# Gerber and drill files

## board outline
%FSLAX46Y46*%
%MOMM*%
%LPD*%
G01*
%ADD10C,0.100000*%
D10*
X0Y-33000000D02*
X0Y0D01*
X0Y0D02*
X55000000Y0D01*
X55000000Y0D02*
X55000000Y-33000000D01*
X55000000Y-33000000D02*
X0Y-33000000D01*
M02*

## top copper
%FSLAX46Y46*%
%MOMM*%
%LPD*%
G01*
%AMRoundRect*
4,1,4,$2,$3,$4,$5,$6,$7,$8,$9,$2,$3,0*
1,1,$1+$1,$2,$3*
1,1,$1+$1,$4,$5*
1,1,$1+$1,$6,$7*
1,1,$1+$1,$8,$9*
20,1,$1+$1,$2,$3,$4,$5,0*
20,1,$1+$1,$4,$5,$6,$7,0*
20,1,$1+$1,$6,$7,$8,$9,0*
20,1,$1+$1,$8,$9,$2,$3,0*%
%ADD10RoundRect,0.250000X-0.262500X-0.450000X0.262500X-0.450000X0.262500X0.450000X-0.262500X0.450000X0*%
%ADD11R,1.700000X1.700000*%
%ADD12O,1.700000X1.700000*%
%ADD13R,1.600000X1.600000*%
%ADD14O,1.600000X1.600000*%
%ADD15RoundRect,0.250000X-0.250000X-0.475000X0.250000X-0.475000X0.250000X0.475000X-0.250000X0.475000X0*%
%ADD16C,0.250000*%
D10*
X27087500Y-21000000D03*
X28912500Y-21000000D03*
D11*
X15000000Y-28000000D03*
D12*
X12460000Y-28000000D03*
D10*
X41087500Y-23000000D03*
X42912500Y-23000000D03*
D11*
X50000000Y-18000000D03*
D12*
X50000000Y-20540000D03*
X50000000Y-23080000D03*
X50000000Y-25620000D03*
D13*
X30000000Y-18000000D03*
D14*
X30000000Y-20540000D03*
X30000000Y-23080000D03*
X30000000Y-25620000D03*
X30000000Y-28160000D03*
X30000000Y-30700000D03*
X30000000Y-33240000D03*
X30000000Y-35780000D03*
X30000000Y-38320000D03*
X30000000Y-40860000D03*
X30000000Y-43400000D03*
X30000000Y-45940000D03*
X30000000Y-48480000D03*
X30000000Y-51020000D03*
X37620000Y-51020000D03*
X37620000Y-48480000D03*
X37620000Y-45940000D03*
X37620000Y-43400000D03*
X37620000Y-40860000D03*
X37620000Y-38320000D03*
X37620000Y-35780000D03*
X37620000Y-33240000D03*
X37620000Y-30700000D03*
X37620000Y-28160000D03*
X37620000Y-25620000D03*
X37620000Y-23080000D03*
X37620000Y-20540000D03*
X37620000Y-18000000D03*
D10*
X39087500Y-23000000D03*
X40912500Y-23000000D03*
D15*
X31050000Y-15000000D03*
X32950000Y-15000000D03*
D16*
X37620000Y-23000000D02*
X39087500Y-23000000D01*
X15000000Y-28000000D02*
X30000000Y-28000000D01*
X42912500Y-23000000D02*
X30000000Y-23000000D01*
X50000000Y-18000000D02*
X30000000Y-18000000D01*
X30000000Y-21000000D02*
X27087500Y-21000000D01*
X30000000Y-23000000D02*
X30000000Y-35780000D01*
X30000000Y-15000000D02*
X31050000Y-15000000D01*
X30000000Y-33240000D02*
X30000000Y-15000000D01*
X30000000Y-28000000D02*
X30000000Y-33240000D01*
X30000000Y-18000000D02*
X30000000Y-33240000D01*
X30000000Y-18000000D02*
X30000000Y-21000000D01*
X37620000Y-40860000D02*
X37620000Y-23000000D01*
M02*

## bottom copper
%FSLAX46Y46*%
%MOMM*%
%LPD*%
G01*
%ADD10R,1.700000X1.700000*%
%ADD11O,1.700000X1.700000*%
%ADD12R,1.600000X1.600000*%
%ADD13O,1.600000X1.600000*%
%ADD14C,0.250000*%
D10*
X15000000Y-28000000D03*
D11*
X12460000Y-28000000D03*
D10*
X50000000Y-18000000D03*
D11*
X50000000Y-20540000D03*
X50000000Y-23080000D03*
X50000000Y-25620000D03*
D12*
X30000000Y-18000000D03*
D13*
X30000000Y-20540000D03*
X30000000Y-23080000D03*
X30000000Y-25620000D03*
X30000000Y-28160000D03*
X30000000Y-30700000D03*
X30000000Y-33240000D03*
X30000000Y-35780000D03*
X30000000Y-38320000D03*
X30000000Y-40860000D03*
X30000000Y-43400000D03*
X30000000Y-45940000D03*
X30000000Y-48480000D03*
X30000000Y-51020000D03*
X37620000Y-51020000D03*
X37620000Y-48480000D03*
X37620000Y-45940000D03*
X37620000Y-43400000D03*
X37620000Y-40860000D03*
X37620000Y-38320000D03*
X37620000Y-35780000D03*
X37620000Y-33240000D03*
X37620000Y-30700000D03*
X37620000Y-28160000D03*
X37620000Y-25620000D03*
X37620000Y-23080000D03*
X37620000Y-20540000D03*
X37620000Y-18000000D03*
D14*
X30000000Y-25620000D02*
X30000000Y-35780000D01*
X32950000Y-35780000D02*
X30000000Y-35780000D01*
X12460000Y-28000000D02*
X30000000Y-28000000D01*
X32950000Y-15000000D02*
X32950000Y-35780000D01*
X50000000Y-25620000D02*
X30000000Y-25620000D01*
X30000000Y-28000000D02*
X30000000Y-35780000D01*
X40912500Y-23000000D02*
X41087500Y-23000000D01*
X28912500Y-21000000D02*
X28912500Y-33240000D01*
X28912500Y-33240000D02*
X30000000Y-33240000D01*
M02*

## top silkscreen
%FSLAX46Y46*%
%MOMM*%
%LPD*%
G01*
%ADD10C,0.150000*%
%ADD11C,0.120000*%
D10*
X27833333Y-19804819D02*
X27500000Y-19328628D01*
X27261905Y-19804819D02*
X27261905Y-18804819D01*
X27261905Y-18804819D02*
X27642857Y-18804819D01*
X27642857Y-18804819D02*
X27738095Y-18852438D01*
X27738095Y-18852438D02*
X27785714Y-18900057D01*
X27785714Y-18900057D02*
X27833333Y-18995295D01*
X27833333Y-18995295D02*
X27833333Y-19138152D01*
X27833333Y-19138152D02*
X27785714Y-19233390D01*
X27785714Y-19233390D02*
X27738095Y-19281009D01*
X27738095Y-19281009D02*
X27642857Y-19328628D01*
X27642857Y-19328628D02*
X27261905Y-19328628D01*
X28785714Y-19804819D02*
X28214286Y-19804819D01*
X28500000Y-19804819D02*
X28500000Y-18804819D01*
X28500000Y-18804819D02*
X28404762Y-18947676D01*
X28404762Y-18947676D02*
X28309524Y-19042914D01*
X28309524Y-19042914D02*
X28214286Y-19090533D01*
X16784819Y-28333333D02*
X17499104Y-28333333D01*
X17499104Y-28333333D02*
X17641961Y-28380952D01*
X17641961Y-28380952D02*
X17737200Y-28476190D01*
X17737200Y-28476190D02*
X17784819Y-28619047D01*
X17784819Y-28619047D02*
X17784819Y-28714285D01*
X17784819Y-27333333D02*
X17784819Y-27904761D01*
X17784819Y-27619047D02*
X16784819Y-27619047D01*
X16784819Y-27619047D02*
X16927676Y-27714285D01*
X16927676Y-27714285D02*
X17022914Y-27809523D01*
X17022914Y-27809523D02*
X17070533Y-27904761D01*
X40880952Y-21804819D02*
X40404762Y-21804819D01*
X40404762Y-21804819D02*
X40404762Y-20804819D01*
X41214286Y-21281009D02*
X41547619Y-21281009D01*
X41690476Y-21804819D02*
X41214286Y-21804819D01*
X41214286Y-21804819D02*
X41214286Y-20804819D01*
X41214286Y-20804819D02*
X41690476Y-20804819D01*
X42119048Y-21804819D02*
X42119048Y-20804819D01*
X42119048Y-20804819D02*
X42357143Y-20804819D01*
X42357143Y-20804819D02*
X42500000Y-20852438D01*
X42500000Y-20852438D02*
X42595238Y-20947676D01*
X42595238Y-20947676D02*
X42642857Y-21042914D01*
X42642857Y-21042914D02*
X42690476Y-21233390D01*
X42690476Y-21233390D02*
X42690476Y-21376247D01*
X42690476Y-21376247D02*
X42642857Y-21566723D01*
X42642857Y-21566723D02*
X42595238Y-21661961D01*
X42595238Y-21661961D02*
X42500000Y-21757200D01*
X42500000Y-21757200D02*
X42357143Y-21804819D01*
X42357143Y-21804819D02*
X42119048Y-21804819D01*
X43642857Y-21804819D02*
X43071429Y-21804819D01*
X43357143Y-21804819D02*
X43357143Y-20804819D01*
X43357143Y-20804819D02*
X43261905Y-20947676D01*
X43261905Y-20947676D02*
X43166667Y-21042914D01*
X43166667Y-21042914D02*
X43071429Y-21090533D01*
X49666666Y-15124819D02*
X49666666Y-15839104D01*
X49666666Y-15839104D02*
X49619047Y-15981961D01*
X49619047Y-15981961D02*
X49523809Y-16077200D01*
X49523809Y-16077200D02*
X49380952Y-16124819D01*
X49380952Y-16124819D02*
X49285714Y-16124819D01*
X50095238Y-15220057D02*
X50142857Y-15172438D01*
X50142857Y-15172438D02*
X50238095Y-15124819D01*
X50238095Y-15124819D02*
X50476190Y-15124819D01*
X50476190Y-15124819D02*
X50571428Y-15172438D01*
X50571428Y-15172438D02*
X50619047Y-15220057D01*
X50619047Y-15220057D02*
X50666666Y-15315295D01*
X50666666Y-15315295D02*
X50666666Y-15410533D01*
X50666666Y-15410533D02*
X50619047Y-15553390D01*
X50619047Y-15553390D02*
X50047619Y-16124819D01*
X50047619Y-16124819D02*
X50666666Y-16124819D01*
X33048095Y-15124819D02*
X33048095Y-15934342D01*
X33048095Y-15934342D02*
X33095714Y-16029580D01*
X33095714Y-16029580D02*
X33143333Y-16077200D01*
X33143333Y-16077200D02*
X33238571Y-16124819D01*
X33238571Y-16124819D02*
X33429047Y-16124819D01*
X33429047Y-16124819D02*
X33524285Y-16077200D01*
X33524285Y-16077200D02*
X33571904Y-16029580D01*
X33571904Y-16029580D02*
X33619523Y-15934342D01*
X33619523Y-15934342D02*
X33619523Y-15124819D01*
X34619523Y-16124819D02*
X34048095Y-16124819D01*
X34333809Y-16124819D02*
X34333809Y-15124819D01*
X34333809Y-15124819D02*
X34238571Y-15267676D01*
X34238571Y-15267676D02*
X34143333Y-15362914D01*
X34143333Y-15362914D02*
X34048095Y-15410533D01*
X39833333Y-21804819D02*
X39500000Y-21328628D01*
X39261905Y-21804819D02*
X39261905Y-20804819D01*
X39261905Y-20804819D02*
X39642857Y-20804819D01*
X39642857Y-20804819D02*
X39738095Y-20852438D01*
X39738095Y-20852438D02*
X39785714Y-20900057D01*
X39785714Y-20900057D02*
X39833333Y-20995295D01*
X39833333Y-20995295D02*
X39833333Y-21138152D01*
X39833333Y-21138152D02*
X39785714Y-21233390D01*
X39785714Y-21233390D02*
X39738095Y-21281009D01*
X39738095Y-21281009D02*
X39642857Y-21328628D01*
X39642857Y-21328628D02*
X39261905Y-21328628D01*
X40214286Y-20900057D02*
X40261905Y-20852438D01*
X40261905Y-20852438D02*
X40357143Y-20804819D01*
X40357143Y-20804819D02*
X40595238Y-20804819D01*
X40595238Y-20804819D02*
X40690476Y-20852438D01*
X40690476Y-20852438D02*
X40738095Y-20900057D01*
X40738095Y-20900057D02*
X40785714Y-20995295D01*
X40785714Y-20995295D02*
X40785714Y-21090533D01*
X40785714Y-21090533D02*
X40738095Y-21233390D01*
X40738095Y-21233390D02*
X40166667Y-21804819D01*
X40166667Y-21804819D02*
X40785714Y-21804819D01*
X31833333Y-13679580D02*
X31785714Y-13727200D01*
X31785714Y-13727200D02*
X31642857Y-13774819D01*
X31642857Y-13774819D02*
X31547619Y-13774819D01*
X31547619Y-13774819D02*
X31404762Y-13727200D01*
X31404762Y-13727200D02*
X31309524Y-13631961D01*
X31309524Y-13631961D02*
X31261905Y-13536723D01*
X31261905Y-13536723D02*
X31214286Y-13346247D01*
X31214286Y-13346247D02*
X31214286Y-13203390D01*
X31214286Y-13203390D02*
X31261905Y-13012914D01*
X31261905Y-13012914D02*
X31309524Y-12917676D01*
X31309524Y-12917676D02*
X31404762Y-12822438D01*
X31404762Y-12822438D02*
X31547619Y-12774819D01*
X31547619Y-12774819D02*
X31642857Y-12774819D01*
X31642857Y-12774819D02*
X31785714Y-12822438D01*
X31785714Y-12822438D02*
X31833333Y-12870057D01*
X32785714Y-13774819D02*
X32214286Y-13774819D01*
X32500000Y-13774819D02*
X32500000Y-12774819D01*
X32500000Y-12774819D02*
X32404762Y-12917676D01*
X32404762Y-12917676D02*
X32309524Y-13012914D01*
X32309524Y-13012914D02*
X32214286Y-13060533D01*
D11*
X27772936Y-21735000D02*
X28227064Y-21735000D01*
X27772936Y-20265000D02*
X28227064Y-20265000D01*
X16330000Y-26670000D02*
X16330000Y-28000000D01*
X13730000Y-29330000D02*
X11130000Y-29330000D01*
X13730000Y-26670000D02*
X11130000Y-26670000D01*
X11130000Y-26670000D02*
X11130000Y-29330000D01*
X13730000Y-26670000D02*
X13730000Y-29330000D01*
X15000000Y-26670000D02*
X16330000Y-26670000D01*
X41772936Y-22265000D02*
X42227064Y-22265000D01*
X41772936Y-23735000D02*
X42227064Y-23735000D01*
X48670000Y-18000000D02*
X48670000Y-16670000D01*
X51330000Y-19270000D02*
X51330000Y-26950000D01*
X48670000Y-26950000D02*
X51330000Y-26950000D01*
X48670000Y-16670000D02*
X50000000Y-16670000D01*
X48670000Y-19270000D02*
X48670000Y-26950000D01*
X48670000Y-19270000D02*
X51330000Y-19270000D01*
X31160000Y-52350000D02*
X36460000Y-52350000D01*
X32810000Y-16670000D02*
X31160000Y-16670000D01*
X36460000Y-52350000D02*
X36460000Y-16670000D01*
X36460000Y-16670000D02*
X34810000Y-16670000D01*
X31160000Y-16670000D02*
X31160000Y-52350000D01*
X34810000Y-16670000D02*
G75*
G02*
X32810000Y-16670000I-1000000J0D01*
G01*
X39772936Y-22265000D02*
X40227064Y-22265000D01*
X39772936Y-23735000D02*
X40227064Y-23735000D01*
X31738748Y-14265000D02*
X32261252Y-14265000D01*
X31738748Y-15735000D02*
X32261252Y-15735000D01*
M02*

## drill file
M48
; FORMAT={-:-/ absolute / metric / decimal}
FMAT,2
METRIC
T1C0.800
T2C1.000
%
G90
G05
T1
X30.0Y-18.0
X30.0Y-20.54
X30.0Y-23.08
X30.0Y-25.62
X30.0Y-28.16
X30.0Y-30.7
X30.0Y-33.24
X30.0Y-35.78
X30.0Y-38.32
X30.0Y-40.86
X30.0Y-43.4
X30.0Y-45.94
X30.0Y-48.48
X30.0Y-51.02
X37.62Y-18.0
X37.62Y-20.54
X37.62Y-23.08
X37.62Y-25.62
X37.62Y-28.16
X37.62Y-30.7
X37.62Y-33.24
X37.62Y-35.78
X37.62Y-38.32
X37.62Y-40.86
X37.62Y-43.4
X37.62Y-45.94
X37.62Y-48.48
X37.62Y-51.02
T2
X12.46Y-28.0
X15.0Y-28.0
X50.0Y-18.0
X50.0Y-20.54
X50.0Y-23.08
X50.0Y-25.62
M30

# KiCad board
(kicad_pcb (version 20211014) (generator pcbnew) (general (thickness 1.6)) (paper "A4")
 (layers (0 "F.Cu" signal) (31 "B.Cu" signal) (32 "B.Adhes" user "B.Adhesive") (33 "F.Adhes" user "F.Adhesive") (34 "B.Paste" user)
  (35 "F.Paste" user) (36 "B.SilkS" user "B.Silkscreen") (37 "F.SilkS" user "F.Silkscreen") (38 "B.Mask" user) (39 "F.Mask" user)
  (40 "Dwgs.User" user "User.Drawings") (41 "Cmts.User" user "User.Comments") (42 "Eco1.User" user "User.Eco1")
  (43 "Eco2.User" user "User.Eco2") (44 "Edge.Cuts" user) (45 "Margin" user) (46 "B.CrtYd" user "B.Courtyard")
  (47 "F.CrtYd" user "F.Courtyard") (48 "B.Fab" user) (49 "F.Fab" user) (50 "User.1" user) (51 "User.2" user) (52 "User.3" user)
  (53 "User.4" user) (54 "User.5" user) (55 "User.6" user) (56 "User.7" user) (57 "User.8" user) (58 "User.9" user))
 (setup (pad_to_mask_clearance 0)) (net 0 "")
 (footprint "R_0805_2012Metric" (layer "F.Cu") (at 28 21)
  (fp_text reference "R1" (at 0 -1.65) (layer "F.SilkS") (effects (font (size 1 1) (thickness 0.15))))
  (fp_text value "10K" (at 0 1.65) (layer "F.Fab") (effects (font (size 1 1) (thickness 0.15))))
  (fp_line (start -0.227064 0.735) (end 0.227064 0.735) (layer "F.SilkS") (width 0.12))
  (fp_line (start -0.227064 -0.735) (end 0.227064 -0.735) (layer "F.SilkS") (width 0.12))
  (pad "1" smd roundrect (at -0.9125 0) (size 1.025 1.4) (layers "F.Cu" "F.Paste" "F.Mask") (roundrect_rratio 0.243902))
  (pad "2" smd roundrect (at 0.9125 0) (size 1.025 1.4) (layers "F.Cu" "F.Paste" "F.Mask") (roundrect_rratio 0.243902)))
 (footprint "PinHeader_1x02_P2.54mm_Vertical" (layer "F.Cu") (at 15 28 -90)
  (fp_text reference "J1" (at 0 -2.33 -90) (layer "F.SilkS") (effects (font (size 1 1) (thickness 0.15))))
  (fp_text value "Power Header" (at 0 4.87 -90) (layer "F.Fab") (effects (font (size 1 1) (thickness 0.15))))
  (fp_line (start -1.33 -1.33) (end 0 -1.33) (layer "F.SilkS") (width 0.12))
  (fp_line (start 1.33 1.27) (end 1.33 3.87) (layer "F.SilkS") (width 0.12))
  (fp_line (start -1.33 1.27) (end -1.33 3.87) (layer "F.SilkS") (width 0.12))
  (fp_line (start -1.33 3.87) (end 1.33 3.87) (layer "F.SilkS") (width 0.12))
  (fp_line (start -1.33 1.27) (end 1.33 1.27) (layer "F.SilkS") (width 0.12))
  (fp_line (start -1.33 0) (end -1.33 -1.33) (layer "F.SilkS") (width 0.12))
  (pad "1" thru_hole rect (at 0 0 270) (size 1.7 1.7) (drill 1) (layers *.Cu *.Mask))
  (pad "2" thru_hole oval (at 0 2.54 270) (size 1.7 1.7) (drill 1) (layers *.Cu *.Mask)))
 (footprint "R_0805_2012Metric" (layer "F.Cu") (at 42 23)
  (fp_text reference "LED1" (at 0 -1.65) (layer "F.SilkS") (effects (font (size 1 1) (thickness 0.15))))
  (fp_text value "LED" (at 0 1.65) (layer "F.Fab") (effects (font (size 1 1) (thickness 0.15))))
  (fp_line (start -0.227064 -0.735) (end 0.227064 -0.735) (layer "F.SilkS") (width 0.12))
  (fp_line (start -0.227064 0.735) (end 0.227064 0.735) (layer "F.SilkS") (width 0.12))
  (pad "1" smd roundrect (at -0.9125 0) (size 1.025 1.4) (layers "F.Cu" "F.Paste" "F.Mask") (roundrect_rratio 0.243902))
  (pad "2" smd roundrect (at 0.9125 0) (size 1.025 1.4) (layers "F.Cu" "F.Paste" "F.Mask") (roundrect_rratio 0.243902)))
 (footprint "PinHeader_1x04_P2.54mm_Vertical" (layer "F.Cu") (at 50 18)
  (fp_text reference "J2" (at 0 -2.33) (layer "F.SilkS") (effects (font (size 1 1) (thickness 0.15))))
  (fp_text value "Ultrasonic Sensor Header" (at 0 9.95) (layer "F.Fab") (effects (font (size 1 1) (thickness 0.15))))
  (fp_line (start -1.33 0) (end -1.33 -1.33) (layer "F.SilkS") (width 0.12))
  (fp_line (start 1.33 1.27) (end 1.33 8.95) (layer "F.SilkS") (width 0.12))
  (fp_line (start -1.33 8.95) (end 1.33 8.95) (layer "F.SilkS") (width 0.12))
  (fp_line (start -1.33 -1.33) (end 0 -1.33) (layer "F.SilkS") (width 0.12))
  (fp_line (start -1.33 1.27) (end -1.33 8.95) (layer "F.SilkS") (width 0.12))
  (fp_line (start -1.33 1.27) (end 1.33 1.27) (layer "F.SilkS") (width 0.12))
  (pad "1" thru_hole rect (at 0 0) (size 1.7 1.7) (drill 1) (layers *.Cu *.Mask))
  (pad "2" thru_hole oval (at 0 2.54) (size 1.7 1.7) (drill 1) (layers *.Cu *.Mask))
  (pad "3" thru_hole oval (at 0 5.08) (size 1.7 1.7) (drill 1) (layers *.Cu *.Mask))
  (pad "4" thru_hole oval (at 0 7.62) (size 1.7 1.7) (drill 1) (layers *.Cu *.Mask)))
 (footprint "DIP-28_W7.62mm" (layer "F.Cu") (at 30 18)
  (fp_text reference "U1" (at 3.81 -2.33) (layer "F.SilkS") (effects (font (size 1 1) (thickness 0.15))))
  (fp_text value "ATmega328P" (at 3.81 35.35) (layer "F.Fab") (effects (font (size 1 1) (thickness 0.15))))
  (fp_line (start 1.16 34.35) (end 6.46 34.35) (layer "F.SilkS") (width 0.12))
  (fp_line (start 2.81 -1.33) (end 1.16 -1.33) (layer "F.SilkS") (width 0.12))
  (fp_line (start 6.46 34.35) (end 6.46 -1.33) (layer "F.SilkS") (width 0.12))
  (fp_line (start 6.46 -1.33) (end 4.81 -1.33) (layer "F.SilkS") (width 0.12))
  (fp_line (start 1.16 -1.33) (end 1.16 34.35) (layer "F.SilkS") (width 0.12))
  (fp_arc (start 4.81 -1.33) (mid 3.81 -0.33) (end 2.81 -1.33) (layer "F.SilkS") (width 0.12))
  (pad "1" thru_hole rect (at 0 0) (size 1.6 1.6) (drill 0.8) (layers *.Cu *.Mask))
  (pad "2" thru_hole oval (at 0 2.54) (size 1.6 1.6) (drill 0.8) (layers *.Cu *.Mask))
  (pad "3" thru_hole oval (at 0 5.08) (size 1.6 1.6) (drill 0.8) (layers *.Cu *.Mask))
  (pad "4" thru_hole oval (at 0 7.62) (size 1.6 1.6) (drill 0.8) (layers *.Cu *.Mask))
  (pad "5" thru_hole oval (at 0 10.16) (size 1.6 1.6) (drill 0.8) (layers *.Cu *.Mask))
  (pad "6" thru_hole oval (at 0 12.7) (size 1.6 1.6) (drill 0.8) (layers *.Cu *.Mask))
  (pad "7" thru_hole oval (at 0 15.24) (size 1.6 1.6) (drill 0.8) (layers *.Cu *.Mask))
  (pad "8" thru_hole oval (at 0 17.78) (size 1.6 1.6) (drill 0.8) (layers *.Cu *.Mask))
  (pad "9" thru_hole oval (at 0 20.32) (size 1.6 1.6) (drill 0.8) (layers *.Cu *.Mask))
  (pad "10" thru_hole oval (at 0 22.86) (size 1.6 1.6) (drill 0.8) (layers *.Cu *.Mask))
  (pad "11" thru_hole oval (at 0 25.4) (size 1.6 1.6) (drill 0.8) (layers *.Cu *.Mask))
  (pad "12" thru_hole oval (at 0 27.94) (size 1.6 1.6) (drill 0.8) (layers *.Cu *.Mask))
  (pad "13" thru_hole oval (at 0 30.48) (size 1.6 1.6) (drill 0.8) (layers *.Cu *.Mask))
  (pad "14" thru_hole oval (at 0 33.02) (size 1.6 1.6) (drill 0.8) (layers *.Cu *.Mask))
  (pad "15" thru_hole oval (at 7.62 33.02) (size 1.6 1.6) (drill 0.8) (layers *.Cu *.Mask))
  (pad "16" thru_hole oval (at 7.62 30.48) (size 1.6 1.6) (drill 0.8) (layers *.Cu *.Mask))
  (pad "17" thru_hole oval (at 7.62 27.94) (size 1.6 1.6) (drill 0.8) (layers *.Cu *.Mask))
  (pad "18" thru_hole oval (at 7.62 25.4) (size 1.6 1.6) (drill 0.8) (layers *.Cu *.Mask))
  (pad "19" thru_hole oval (at 7.62 22.86) (size 1.6 1.6) (drill 0.8) (layers *.Cu *.Mask))
  (pad "20" thru_hole oval (at 7.62 20.32) (size 1.6 1.6) (drill 0.8) (layers *.Cu *.Mask))
  (pad "21" thru_hole oval (at 7.62 17.78) (size 1.6 1.6) (drill 0.8) (layers *.Cu *.Mask))
  (pad "22" thru_hole oval (at 7.62 15.24) (size 1.6 1.6) (drill 0.8) (layers *.Cu *.Mask))
  (pad "23" thru_hole oval (at 7.62 12.7) (size 1.6 1.6) (drill 0.8) (layers *.Cu *.Mask))
  (pad "24" thru_hole oval (at 7.62 10.16) (size 1.6 1.6) (drill 0.8) (layers *.Cu *.Mask))
  (pad "25" thru_hole oval (at 7.62 7.62) (size 1.6 1.6) (drill 0.8) (layers *.Cu *.Mask))
  (pad "26" thru_hole oval (at 7.62 5.08) (size 1.6 1.6) (drill 0.8) (layers *.Cu *.Mask))
  (pad "27" thru_hole oval (at 7.62 2.54) (size 1.6 1.6) (drill 0.8) (layers *.Cu *.Mask))
  (pad "28" thru_hole oval (at 7.62 0) (size 1.6 1.6) (drill 0.8) (layers *.Cu *.Mask)))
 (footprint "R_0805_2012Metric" (layer "F.Cu") (at 40 23)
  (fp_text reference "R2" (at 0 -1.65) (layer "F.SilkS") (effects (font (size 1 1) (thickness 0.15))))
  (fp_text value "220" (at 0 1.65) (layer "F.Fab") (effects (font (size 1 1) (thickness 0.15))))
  (fp_line (start -0.227064 -0.735) (end 0.227064 -0.735) (layer "F.SilkS") (width 0.12))
  (fp_line (start -0.227064 0.735) (end 0.227064 0.735) (layer "F.SilkS") (width 0.12))
  (pad "1" smd roundrect (at -0.9125 0) (size 1.025 1.4) (layers "F.Cu" "F.Paste" "F.Mask") (roundrect_rratio 0.243902))
  (pad "2" smd roundrect (at 0.9125 0) (size 1.025 1.4) (layers "F.Cu" "F.Paste" "F.Mask") (roundrect_rratio 0.243902)))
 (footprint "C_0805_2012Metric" (layer "F.Cu") (at 32 15)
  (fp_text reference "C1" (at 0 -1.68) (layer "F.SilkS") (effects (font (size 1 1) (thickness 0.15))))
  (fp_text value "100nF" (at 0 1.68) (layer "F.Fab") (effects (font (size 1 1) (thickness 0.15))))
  (fp_line (start -0.261252 -0.735) (end 0.261252 -0.735) (layer "F.SilkS") (width 0.12))
  (fp_line (start -0.261252 0.735) (end 0.261252 0.735) (layer "F.SilkS") (width 0.12))
  (pad "1" smd roundrect (at -0.95 0) (size 1 1.45) (layers "F.Cu" "F.Paste" "F.Mask") (roundrect_rratio 0.25))
  (pad "2" smd roundrect (at 0.95 0) (size 1 1.45) (layers "F.Cu" "F.Paste" "F.Mask") (roundrect_rratio 0.25)))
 (gr_line (start 0 33) (end 0 0) (layer "Edge.Cuts") (width 0.1))
 (gr_line (start 0 0) (end 55 0) (layer "Edge.Cuts") (width 0.1))
 (gr_line (start 55 0) (end 55 33) (layer "Edge.Cuts") (width 0.1))
 (gr_line (start 55 33) (end 0 33) (layer "Edge.Cuts") (width 0.1))
 (segment (start 37.62 23) (end 39.0875 23) (width 0.25) (layer "F.Cu") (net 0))
 (segment (start 15 28) (end 30 28) (width 0.25) (layer "F.Cu") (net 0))
 (segment (start 42.9125 23) (end 30 23) (width 0.25) (layer "F.Cu") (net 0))
 (segment (start 50 18) (end 30 18) (width 0.25) (layer "F.Cu") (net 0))
 (segment (start 30 21) (end 27.0875 21) (width 0.25) (layer "F.Cu") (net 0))
 (segment (start 30 23) (end 30 35.78) (width 0.25) (layer "F.Cu") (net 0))
 (segment (start 30 15) (end 31.05 15) (width 0.25) (layer "F.Cu") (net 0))
 (segment (start 30 33.24) (end 30 15) (width 0.25) (layer "F.Cu") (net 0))
 (segment (start 30 28) (end 30 33.24) (width 0.25) (layer "F.Cu") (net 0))
 (segment (start 30 18) (end 30 33.24) (width 0.25) (layer "F.Cu") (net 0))
 (segment (start 30 18) (end 30 21) (width 0.25) (layer "F.Cu") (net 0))
 (segment (start 37.62 40.86) (end 37.62 23) (width 0.25) (layer "F.Cu") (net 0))
 (segment (start 30 25.62) (end 30 35.78) (width 0.25) (layer "B.Cu") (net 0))
 (segment (start 32.95 35.78) (end 30 35.78) (width 0.25) (layer "B.Cu") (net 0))
 (segment (start 12.46 28) (end 30 28) (width 0.25) (layer "B.Cu") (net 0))
 (segment (start 32.95 15) (end 32.95 35.78) (width 0.25) (layer "B.Cu") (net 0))
 (segment (start 50 25.62) (end 30 25.62) (width 0.25) (layer "B.Cu") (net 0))
 (segment (start 30 28) (end 30 35.78) (width 0.25) (layer "B.Cu") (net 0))
 (segment (start 40.9125 23) (end 41.0875 23) (width 0.25) (layer "B.Cu") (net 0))
 (segment (start 28.9125 21) (end 28.9125 33.24) (width 0.25) (layer "B.Cu") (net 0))
 (segment (start 28.9125 33.24) (end 30 33.24) (width 0.25) (layer "B.Cu") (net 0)))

